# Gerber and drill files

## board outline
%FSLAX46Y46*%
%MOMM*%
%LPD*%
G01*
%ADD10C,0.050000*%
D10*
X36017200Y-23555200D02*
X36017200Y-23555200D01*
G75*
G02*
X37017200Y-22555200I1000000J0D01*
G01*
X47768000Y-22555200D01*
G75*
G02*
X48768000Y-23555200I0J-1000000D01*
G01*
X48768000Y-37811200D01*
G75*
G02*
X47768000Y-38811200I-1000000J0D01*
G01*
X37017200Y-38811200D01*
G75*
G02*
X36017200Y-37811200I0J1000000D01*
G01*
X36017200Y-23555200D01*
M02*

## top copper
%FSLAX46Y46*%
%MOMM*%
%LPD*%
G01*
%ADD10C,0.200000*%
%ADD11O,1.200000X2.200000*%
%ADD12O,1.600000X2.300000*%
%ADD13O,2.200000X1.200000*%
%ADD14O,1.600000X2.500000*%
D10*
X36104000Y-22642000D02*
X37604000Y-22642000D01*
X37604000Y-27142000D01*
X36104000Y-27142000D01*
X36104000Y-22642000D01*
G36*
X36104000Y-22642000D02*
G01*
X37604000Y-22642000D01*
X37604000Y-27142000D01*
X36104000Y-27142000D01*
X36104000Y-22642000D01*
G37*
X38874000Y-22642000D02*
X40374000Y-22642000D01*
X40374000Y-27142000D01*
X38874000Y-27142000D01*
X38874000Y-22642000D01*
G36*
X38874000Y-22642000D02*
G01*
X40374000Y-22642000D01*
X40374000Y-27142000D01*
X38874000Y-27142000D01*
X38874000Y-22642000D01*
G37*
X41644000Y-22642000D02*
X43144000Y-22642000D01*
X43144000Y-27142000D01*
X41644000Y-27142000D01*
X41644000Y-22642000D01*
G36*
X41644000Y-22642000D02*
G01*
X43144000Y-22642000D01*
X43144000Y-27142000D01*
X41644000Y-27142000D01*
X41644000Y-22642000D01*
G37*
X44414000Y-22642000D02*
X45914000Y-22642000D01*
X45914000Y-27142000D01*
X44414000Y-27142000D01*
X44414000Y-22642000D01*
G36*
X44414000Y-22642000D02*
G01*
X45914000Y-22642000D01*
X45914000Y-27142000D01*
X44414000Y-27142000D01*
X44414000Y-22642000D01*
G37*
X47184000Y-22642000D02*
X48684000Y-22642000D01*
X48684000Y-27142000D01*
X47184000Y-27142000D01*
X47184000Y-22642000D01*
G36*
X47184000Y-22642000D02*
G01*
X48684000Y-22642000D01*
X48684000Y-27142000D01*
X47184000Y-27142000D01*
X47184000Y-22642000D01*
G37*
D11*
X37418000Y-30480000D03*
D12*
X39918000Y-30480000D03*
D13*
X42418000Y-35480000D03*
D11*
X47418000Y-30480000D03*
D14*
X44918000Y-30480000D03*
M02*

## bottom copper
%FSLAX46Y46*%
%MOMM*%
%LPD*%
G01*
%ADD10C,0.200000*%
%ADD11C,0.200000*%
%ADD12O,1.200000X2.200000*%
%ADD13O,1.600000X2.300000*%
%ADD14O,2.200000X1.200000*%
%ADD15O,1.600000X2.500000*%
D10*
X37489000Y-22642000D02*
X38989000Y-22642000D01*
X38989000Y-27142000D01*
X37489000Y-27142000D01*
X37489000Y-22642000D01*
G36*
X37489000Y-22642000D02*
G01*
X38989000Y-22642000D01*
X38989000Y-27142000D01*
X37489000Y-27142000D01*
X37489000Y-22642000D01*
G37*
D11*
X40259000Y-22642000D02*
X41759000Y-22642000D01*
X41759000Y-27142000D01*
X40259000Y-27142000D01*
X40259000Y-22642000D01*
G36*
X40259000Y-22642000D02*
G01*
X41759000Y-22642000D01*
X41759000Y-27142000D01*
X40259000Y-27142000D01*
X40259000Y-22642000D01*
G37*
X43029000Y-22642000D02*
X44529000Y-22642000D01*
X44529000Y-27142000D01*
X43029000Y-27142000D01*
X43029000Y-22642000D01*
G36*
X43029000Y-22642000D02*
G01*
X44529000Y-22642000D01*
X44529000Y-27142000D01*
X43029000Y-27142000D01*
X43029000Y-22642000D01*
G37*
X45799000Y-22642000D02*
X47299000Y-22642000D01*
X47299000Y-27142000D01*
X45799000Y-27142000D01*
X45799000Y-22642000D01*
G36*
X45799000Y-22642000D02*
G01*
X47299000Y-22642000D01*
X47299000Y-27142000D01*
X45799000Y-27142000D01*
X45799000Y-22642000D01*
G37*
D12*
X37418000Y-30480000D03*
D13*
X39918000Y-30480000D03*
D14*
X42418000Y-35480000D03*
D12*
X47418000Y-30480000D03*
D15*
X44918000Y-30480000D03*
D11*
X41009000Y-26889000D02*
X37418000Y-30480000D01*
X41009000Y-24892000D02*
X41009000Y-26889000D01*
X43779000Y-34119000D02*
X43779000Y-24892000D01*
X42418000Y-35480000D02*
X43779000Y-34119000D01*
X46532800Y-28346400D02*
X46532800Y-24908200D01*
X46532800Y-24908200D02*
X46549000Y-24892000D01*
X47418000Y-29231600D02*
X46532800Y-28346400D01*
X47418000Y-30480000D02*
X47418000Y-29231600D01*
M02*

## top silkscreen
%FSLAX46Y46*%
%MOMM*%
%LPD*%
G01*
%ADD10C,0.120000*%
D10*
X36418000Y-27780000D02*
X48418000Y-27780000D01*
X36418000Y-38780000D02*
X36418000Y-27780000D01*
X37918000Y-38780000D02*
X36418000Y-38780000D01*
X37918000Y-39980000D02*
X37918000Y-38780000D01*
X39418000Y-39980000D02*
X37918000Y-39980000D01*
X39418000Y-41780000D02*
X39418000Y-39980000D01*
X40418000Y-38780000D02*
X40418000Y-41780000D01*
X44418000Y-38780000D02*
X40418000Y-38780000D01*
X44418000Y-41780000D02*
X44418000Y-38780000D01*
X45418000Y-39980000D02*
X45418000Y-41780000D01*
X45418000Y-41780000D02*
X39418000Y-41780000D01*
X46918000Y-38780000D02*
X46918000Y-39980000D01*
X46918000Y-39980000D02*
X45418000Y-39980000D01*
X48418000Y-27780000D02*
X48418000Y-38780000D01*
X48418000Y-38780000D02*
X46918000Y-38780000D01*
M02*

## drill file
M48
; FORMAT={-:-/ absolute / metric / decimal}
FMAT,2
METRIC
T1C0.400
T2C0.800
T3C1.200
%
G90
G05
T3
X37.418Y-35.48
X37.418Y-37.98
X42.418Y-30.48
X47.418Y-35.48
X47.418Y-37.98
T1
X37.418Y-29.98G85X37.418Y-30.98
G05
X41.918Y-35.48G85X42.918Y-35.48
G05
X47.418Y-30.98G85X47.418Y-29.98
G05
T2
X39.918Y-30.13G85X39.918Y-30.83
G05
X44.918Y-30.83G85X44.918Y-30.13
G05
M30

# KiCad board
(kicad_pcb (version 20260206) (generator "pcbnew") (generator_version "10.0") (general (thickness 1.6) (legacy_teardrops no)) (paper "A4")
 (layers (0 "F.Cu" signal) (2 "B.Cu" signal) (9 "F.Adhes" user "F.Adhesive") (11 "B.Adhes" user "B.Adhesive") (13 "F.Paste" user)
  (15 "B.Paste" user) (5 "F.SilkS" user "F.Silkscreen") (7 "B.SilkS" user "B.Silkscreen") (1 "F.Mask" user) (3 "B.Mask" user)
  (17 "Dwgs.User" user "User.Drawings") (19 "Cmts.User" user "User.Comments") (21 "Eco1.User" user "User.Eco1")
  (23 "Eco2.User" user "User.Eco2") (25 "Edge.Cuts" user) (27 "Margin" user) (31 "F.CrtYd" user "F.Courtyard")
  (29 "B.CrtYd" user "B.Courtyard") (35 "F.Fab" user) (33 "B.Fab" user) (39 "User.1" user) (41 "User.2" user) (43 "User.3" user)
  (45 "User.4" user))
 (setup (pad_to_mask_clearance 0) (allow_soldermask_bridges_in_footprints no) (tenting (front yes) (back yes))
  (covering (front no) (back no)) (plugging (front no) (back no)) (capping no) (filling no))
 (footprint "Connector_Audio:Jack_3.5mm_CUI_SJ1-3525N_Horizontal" (layer "F.Cu") (at 42.418 35.48)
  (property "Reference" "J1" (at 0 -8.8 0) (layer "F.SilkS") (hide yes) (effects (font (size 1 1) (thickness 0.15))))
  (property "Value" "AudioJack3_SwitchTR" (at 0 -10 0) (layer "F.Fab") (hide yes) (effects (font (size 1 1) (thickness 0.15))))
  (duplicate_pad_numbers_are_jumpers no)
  (fp_line (start -6 -7.7) (end 6 -7.7) (stroke (width 0.12) (type solid)) (layer "F.SilkS"))
  (fp_line (start -6 3.3) (end -6 -7.7) (stroke (width 0.12) (type solid)) (layer "F.SilkS"))
  (fp_line (start -4.5 3.3) (end -6 3.3) (stroke (width 0.12) (type solid)) (layer "F.SilkS"))
  (fp_line (start -4.5 4.5) (end -4.5 3.3) (stroke (width 0.12) (type solid)) (layer "F.SilkS"))
  (fp_line (start -3 4.5) (end -4.5 4.5) (stroke (width 0.12) (type solid)) (layer "F.SilkS"))
  (fp_line (start -3 6.3) (end -3 4.5) (stroke (width 0.12) (type solid)) (layer "F.SilkS"))
  (fp_line (start -2 3.3) (end -2 6.3) (stroke (width 0.12) (type solid)) (layer "F.SilkS"))
  (fp_line (start 2 3.3) (end -2 3.3) (stroke (width 0.12) (type solid)) (layer "F.SilkS"))
  (fp_line (start 2 6.3) (end 2 3.3) (stroke (width 0.12) (type solid)) (layer "F.SilkS"))
  (fp_line (start 3 4.5) (end 3 6.3) (stroke (width 0.12) (type solid)) (layer "F.SilkS"))
  (fp_line (start 3 6.3) (end -3 6.3) (stroke (width 0.12) (type solid)) (layer "F.SilkS"))
  (fp_line (start 4.5 3.3) (end 4.5 4.5) (stroke (width 0.12) (type solid)) (layer "F.SilkS"))
  (fp_line (start 4.5 4.5) (end 3 4.5) (stroke (width 0.12) (type solid)) (layer "F.SilkS"))
  (fp_line (start 6 -7.7) (end 6 3.3) (stroke (width 0.12) (type solid)) (layer "F.SilkS"))
  (fp_line (start 6 3.3) (end 4.5 3.3) (stroke (width 0.12) (type solid)) (layer "F.SilkS"))
  (pad "" np_thru_hole circle (at -5 0) (size 1.2 1.2) (drill 1.2) (layers "*.Cu" "*.Mask"))
  (pad "" np_thru_hole circle (at -5 2.5) (size 1.2 1.2) (drill 1.2) (layers "*.Cu" "*.Mask"))
  (pad "" np_thru_hole circle (at 0 -5) (size 1.2 1.2) (drill 1.2) (layers "*.Cu" "*.Mask"))
  (pad "" np_thru_hole circle (at 5 0) (size 1.2 1.2) (drill 1.2) (layers "*.Cu" "*.Mask"))
  (pad "" np_thru_hole circle (at 5 2.5) (size 1.2 1.2) (drill 1.2) (layers "*.Cu" "*.Mask"))
  (pad "R" thru_hole oval (at -5 -5) (size 1.2 2.2) (drill oval 0.4 1.4) (layers "*.Cu" "*.Mask") (remove_unused_layers no)
   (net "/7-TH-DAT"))
  (pad "RN" thru_hole oval (at -2.5 -5) (size 1.6 2.3) (drill oval 0.8 1.5) (layers "*.Cu" "*.Mask") (remove_unused_layers no)
   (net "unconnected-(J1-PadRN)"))
  (pad "S" thru_hole oval (at 0 0) (size 2.2 1.2) (drill oval 1.4 0.4) (layers "*.Cu" "*.Mask") (remove_unused_layers no) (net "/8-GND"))
  (pad "T" thru_hole oval (at 5 -5 180) (size 1.2 2.2) (drill oval 0.4 1.4) (layers "*.Cu" "*.Mask") (remove_unused_layers no)
   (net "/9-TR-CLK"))
  (pad "TN" thru_hole oval (at 2.5 -5 180) (size 1.6 2.5) (drill oval 0.8 1.5) (layers "*.Cu" "*.Mask") (remove_unused_layers no)
   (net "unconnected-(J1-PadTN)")))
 (gr_rect (start 36.104 22.642) (end 37.604 27.142) (stroke (width 0.2) (type solid)) (fill yes) (layer "F.Cu"))
 (gr_rect (start 38.874 22.642) (end 40.374 27.142) (stroke (width 0.2) (type solid)) (fill yes) (layer "F.Cu"))
 (gr_rect (start 41.644 22.642) (end 43.144 27.142) (stroke (width 0.2) (type solid)) (fill yes) (layer "F.Cu"))
 (gr_rect (start 44.414 22.642) (end 45.914 27.142) (stroke (width 0.2) (type solid)) (fill yes) (layer "F.Cu"))
 (gr_rect (start 47.184 22.642) (end 48.684 27.142) (stroke (width 0.2) (type solid)) (fill yes) (layer "F.Cu"))
 (gr_rect (start 37.489 22.642) (end 38.989 27.142) (stroke (width 0.2) (type solid)) (fill yes) (layer "B.Cu"))
 (gr_rect (start 40.259 22.642) (end 41.759 27.142) (stroke (width 0.2) (type solid)) (fill yes) (layer "B.Cu") (net "/7-TH-DAT"))
 (gr_rect (start 43.029 22.642) (end 44.529 27.142) (stroke (width 0.2) (type solid)) (fill yes) (layer "B.Cu") (net "/8-GND"))
 (gr_rect (start 45.799 22.642) (end 47.299 27.142) (stroke (width 0.2) (type solid)) (fill yes) (layer "B.Cu") (net "/9-TR-CLK"))
 (gr_rect (start 36.0172 22.5552) (end 48.768 38.8112) (radius 1) (stroke (width 0.05) (type solid)) (fill no) (layer "Edge.Cuts"))
 (segment (start 41.009 26.889) (end 37.418 30.48) (width 0.2) (layer "B.Cu") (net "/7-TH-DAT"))
 (segment (start 41.009 24.892) (end 41.009 26.889) (width 0.2) (layer "B.Cu") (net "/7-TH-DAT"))
 (segment (start 43.779 34.119) (end 43.779 24.892) (width 0.2) (layer "B.Cu") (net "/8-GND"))
 (segment (start 42.418 35.48) (end 43.779 34.119) (width 0.2) (layer "B.Cu") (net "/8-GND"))
 (segment (start 46.5328 28.3464) (end 46.5328 24.9082) (width 0.2) (layer "B.Cu") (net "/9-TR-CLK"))
 (segment (start 46.5328 24.9082) (end 46.549 24.892) (width 0.2) (layer "B.Cu") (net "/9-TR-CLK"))
 (segment (start 47.418 29.2316) (end 46.5328 28.3464) (width 0.2) (layer "B.Cu") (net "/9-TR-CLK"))
 (segment (start 47.418 30.48) (end 47.418 29.2316) (width 0.2) (layer "B.Cu") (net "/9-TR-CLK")))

